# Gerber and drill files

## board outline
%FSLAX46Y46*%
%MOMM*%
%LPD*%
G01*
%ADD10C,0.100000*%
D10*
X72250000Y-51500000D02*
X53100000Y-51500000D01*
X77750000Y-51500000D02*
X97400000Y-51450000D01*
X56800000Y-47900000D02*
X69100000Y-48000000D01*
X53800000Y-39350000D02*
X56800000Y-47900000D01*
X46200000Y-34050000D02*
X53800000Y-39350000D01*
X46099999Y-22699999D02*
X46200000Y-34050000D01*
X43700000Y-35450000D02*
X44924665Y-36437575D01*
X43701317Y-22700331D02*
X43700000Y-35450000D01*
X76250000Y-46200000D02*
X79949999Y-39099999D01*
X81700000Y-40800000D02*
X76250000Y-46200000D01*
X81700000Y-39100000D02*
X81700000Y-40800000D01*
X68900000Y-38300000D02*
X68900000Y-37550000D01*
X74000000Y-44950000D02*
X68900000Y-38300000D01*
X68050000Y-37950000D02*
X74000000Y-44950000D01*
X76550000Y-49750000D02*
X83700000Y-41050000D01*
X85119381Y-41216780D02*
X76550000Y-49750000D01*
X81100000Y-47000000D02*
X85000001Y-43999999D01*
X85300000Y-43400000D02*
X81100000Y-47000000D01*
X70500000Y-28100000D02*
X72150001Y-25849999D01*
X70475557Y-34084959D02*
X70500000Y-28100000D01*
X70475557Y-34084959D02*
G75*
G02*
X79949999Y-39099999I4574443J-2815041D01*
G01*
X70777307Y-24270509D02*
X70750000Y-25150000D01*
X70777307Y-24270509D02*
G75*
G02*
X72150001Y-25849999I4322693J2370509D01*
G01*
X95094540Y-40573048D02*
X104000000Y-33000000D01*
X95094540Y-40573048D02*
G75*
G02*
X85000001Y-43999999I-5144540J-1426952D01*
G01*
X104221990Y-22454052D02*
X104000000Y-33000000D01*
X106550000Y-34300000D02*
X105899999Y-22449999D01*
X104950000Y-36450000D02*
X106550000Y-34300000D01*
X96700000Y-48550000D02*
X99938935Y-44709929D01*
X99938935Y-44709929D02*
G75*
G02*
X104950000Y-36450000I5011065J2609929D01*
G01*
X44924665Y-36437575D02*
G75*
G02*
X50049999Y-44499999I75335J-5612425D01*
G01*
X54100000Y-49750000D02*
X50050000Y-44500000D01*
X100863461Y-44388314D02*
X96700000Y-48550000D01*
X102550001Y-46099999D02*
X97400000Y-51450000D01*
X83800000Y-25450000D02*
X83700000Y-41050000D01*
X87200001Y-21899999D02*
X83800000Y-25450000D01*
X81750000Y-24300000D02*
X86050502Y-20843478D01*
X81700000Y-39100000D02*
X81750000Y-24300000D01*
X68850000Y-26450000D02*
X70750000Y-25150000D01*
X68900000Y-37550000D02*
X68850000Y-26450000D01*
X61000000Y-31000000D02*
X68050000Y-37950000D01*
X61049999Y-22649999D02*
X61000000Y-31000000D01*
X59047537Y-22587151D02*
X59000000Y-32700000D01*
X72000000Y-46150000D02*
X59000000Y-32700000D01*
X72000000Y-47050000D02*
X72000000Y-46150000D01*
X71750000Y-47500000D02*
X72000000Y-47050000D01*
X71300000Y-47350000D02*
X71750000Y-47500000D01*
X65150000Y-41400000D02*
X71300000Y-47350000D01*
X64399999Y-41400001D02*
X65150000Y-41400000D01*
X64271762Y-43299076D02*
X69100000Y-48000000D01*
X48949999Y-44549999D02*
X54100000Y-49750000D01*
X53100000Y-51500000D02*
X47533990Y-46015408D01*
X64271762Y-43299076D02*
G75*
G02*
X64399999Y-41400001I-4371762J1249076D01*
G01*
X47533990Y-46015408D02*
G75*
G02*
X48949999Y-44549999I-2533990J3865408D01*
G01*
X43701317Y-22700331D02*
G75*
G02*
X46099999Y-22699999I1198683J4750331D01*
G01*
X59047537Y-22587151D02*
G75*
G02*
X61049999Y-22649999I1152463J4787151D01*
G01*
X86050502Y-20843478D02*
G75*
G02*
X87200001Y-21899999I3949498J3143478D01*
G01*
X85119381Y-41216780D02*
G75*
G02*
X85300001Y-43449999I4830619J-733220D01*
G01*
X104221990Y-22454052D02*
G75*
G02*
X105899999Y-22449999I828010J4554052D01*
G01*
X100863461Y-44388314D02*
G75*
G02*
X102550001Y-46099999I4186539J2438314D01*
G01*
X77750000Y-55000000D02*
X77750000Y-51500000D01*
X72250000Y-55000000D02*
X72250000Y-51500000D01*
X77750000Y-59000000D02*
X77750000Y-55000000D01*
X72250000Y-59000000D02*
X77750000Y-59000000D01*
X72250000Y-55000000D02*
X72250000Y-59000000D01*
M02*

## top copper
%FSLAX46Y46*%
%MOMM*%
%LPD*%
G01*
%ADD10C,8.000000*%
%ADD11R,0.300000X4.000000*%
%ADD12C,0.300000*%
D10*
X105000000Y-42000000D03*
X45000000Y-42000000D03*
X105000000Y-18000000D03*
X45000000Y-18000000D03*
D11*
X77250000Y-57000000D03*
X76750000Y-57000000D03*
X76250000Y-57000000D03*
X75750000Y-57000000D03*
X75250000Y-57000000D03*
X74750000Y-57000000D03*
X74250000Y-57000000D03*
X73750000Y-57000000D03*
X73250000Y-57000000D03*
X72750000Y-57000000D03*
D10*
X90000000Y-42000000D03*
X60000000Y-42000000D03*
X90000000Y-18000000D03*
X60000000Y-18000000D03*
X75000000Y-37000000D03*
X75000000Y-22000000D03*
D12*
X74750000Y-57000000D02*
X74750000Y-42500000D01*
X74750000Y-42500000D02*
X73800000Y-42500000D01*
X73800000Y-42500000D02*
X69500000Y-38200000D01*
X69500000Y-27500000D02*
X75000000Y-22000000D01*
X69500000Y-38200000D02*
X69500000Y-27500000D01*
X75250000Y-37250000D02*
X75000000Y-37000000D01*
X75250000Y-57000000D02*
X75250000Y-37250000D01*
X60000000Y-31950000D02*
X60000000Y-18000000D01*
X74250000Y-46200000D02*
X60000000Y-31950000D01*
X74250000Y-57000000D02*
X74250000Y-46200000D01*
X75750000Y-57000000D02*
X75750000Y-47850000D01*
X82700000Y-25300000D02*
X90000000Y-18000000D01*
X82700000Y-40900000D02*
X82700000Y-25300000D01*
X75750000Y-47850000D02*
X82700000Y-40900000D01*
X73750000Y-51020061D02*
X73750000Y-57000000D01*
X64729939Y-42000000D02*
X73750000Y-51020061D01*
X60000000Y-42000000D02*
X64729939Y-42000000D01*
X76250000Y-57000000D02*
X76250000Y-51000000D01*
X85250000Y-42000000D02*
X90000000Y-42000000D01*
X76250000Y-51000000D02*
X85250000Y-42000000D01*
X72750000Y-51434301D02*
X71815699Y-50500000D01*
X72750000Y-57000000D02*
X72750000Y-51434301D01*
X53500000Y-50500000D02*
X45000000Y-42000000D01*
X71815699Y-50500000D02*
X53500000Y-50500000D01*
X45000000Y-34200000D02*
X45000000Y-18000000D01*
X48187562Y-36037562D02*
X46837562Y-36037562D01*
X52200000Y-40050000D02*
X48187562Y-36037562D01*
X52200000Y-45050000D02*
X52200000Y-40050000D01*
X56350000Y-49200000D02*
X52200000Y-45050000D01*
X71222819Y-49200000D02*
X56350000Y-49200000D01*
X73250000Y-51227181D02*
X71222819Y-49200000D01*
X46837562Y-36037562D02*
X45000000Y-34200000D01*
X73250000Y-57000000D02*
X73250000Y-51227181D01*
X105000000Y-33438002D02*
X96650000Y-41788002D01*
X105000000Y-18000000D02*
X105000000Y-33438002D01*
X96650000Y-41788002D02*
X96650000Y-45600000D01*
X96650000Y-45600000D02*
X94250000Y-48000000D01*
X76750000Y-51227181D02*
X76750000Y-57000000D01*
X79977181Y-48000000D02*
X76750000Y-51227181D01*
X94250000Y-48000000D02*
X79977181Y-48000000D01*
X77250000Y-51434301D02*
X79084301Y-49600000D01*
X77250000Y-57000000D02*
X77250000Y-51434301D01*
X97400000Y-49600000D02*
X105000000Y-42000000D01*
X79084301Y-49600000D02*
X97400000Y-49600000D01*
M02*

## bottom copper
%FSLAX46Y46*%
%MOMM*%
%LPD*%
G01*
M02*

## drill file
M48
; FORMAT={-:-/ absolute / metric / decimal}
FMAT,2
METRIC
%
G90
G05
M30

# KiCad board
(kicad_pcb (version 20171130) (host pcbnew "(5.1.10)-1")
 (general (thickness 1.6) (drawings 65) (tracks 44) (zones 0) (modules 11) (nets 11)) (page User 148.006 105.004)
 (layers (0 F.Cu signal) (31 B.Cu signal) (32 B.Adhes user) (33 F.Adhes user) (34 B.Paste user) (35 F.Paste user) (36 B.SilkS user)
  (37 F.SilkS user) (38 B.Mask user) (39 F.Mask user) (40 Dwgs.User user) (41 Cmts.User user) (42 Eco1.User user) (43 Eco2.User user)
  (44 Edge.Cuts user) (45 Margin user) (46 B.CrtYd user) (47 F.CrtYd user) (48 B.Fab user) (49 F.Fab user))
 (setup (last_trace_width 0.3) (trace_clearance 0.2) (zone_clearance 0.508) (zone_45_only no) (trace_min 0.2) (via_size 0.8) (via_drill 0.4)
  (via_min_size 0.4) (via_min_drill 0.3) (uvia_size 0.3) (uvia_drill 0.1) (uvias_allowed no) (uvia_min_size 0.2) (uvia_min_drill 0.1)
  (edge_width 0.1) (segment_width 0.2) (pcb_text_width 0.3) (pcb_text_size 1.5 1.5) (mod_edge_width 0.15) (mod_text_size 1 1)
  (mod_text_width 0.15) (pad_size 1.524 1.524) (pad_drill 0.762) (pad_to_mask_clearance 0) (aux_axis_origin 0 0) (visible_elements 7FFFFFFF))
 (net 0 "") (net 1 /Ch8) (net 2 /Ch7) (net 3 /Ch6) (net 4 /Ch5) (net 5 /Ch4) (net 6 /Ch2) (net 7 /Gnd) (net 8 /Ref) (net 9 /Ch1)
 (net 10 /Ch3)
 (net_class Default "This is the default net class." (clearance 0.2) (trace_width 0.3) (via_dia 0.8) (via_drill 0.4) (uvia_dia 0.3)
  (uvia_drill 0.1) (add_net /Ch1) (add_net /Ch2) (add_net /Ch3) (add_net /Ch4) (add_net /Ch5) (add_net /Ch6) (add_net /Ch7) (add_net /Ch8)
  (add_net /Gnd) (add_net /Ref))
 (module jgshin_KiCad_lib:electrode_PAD (layer F.Cu) (at 105 42)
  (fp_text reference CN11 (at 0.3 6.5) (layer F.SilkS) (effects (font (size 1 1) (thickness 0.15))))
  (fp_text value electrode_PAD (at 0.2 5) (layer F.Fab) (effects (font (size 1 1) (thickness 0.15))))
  (pad 1 smd circle (at 0 0) (size 8 8) (layers F.Cu F.Paste F.Mask) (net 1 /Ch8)))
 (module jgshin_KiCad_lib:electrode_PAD (layer F.Cu) (at 45 42)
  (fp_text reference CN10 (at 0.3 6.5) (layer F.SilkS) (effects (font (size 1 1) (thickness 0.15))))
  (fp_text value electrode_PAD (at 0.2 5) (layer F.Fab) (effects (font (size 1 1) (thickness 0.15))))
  (pad 1 smd circle (at 0 0) (size 8 8) (layers F.Cu F.Paste F.Mask) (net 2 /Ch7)))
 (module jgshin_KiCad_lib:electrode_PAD (layer F.Cu) (at 105 18)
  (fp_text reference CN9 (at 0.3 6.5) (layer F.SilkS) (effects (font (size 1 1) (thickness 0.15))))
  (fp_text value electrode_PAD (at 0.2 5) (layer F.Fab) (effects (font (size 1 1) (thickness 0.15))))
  (pad 1 smd circle (at 0 0) (size 8 8) (layers F.Cu F.Paste F.Mask) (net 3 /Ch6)))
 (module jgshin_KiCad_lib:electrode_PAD (layer F.Cu) (at 45 18)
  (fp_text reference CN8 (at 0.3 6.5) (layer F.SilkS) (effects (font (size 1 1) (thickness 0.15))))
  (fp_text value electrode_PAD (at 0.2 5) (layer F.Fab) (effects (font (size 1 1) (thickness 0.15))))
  (pad 1 smd circle (at 0 0) (size 8 8) (layers F.Cu F.Paste F.Mask) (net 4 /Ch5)))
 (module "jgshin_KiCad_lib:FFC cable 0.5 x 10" (layer F.Cu) (at 75 57)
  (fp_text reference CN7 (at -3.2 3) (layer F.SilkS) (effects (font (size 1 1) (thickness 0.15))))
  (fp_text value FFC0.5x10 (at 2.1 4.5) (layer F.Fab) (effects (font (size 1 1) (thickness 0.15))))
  (pad 10 smd rect (at 2.25 0) (size 0.3 4) (layers F.Cu F.Paste F.Mask) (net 1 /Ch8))
  (pad 9 smd rect (at 1.75 0) (size 0.3 4) (layers F.Cu F.Paste F.Mask) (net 3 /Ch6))
  (pad 8 smd rect (at 1.25 0) (size 0.3 4) (layers F.Cu F.Paste F.Mask) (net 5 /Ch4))
  (pad 7 smd rect (at 0.75 0) (size 0.3 4) (layers F.Cu F.Paste F.Mask) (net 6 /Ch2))
  (pad 6 smd rect (at 0.25 0) (size 0.3 4) (layers F.Cu F.Paste F.Mask) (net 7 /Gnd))
  (pad 5 smd rect (at -0.25 0) (size 0.3 4) (layers F.Cu F.Paste F.Mask) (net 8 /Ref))
  (pad 4 smd rect (at -0.75 0) (size 0.3 4) (layers F.Cu F.Paste F.Mask) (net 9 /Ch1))
  (pad 3 smd rect (at -1.25 0) (size 0.3 4) (layers F.Cu F.Paste F.Mask) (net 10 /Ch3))
  (pad 2 smd rect (at -1.75 0) (size 0.3 4) (layers F.Cu F.Paste F.Mask) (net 4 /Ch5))
  (pad 1 smd rect (at -2.25 0) (size 0.3 4) (layers F.Cu F.Paste F.Mask) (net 2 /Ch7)))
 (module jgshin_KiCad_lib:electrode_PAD (layer F.Cu) (at 90 42)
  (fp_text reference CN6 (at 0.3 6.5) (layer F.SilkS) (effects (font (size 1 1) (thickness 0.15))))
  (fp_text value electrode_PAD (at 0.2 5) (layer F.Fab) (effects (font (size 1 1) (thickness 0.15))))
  (pad 1 smd circle (at 0 0) (size 8 8) (layers F.Cu F.Paste F.Mask) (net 5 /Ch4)))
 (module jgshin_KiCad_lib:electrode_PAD (layer F.Cu) (at 60 42)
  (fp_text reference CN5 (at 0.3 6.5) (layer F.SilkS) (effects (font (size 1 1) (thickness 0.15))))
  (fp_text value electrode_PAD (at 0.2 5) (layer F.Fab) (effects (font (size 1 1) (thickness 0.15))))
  (pad 1 smd circle (at 0 0) (size 8 8) (layers F.Cu F.Paste F.Mask) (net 10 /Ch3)))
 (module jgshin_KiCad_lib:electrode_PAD (layer F.Cu) (at 90 18)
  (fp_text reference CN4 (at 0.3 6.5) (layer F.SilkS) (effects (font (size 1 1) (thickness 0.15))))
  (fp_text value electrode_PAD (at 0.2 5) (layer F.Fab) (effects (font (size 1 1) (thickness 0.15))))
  (pad 1 smd circle (at 0 0) (size 8 8) (layers F.Cu F.Paste F.Mask) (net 6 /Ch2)))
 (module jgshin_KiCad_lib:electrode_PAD (layer F.Cu) (at 60 18)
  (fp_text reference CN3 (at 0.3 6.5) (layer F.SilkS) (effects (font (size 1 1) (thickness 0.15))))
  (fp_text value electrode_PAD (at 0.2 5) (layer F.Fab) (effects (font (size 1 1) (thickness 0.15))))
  (pad 1 smd circle (at 0 0) (size 8 8) (layers F.Cu F.Paste F.Mask) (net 9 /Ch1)))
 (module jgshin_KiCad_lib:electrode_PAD (layer F.Cu) (at 75 37)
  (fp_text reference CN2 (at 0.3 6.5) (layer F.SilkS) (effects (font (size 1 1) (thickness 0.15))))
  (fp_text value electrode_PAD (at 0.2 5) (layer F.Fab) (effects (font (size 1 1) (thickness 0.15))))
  (pad 1 smd circle (at 0 0) (size 8 8) (layers F.Cu F.Paste F.Mask) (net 7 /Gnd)))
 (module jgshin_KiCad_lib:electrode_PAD (layer F.Cu) (at 75 22)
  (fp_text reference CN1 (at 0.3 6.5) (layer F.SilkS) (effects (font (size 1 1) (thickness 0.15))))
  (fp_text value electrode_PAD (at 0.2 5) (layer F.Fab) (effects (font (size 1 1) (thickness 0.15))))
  (pad 1 smd circle (at 0 0) (size 8 8) (layers F.Cu F.Paste F.Mask) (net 8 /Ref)))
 (gr_line (start 72.25 51.5) (end 53.1 51.5) (layer Edge.Cuts) (width 0.1))
 (gr_line (start 77.75 51.5) (end 97.4 51.45) (layer Edge.Cuts) (width 0.1))
 (gr_line (start 56.8 47.9) (end 69.1 48) (layer Edge.Cuts) (width 0.1))
 (gr_line (start 53.8 39.35) (end 56.8 47.9) (layer Edge.Cuts) (width 0.1))
 (gr_line (start 46.2 34.05) (end 53.8 39.35) (layer Edge.Cuts) (width 0.1))
 (gr_line (start 46.099999 22.699999) (end 46.2 34.05) (layer Edge.Cuts) (width 0.1))
 (gr_line (start 43.7 35.45) (end 44.924665 36.437575) (layer Edge.Cuts) (width 0.1))
 (gr_line (start 43.701317 22.700331) (end 43.7 35.45) (layer Edge.Cuts) (width 0.1))
 (gr_line (start 76.25 46.2) (end 79.949999 39.099999) (layer Edge.Cuts) (width 0.1))
 (gr_line (start 81.7 40.8) (end 76.25 46.2) (layer Edge.Cuts) (width 0.1))
 (gr_line (start 81.7 39.1) (end 81.7 40.8) (layer Edge.Cuts) (width 0.1))
 (gr_line (start 68.9 38.3) (end 68.9 37.55) (layer Edge.Cuts) (width 0.1))
 (gr_line (start 74 44.95) (end 68.9 38.3) (layer Edge.Cuts) (width 0.1))
 (gr_line (start 68.05 37.95) (end 74 44.95) (layer Edge.Cuts) (width 0.1))
 (gr_line (start 76.55 49.75) (end 83.7 41.05) (layer Edge.Cuts) (width 0.1))
 (gr_line (start 85.119381 41.21678) (end 76.55 49.75) (layer Edge.Cuts) (width 0.1))
 (gr_line (start 81.1 47) (end 85.000001 43.999999) (layer Edge.Cuts) (width 0.1))
 (gr_line (start 85.3 43.4) (end 81.1 47) (layer Edge.Cuts) (width 0.1))
 (gr_line (start 70.5 28.1) (end 72.150001 25.849999) (layer Edge.Cuts) (width 0.1))
 (gr_line (start 70.475557 34.084959) (end 70.5 28.1) (layer Edge.Cuts) (width 0.1))
 (gr_arc (start 75.05 36.9) (end 79.949999 39.099999) (angle -172.5716049) (layer Edge.Cuts) (width 0.1))
 (gr_line (start 70.777307 24.270509) (end 70.75 25.15) (layer Edge.Cuts) (width 0.1))
 (gr_arc (start 75.1 21.9) (end 72.150001 25.849999) (angle -335.4934745) (layer Edge.Cuts) (width 0.1))
 (gr_line (start 95.09454 40.573048) (end 104 33) (layer Edge.Cuts) (width 0.1))
 (gr_arc (start 89.95 42) (end 85.000001 43.999999) (angle -173.5018404) (layer Edge.Cuts) (width 0.1))
 (gr_line (start 104.22199 22.454052) (end 104 33) (layer Edge.Cuts) (width 0.1))
 (gr_line (start 106.55 34.3) (end 105.899999 22.449999) (layer Edge.Cuts) (width 0.1))
 (gr_line (start 104.95 36.45) (end 106.55 34.3) (layer Edge.Cuts) (width 0.1))
 (gr_line (start 96.7 48.55) (end 99.938935 44.709929) (layer Edge.Cuts) (width 0.1))
 (gr_arc (start 104.95 42.1) (end 104.95 36.45) (angle -117.5120026) (layer Edge.Cuts) (width 0.1))
 (gr_arc (start 45 42.05) (end 50.049999 44.499999) (angle -116.6492984) (layer Edge.Cuts) (width 0.1))
 (gr_line (start 54.1 49.75) (end 50.05 44.5) (layer Edge.Cuts) (width 0.1))
 (gr_line (start 100.863461 44.388314) (end 96.7 48.55) (layer Edge.Cuts) (width 0.1))
 (gr_line (start 102.550001 46.099999) (end 97.4 51.45) (layer Edge.Cuts) (width 0.1))
 (gr_line (start 83.8 25.45) (end 83.7 41.05) (layer Edge.Cuts) (width 0.1))
 (gr_line (start 87.200001 21.899999) (end 83.8 25.45) (layer Edge.Cuts) (width 0.1))
 (gr_line (start 81.75 24.3) (end 86.050502 20.843478) (layer Edge.Cuts) (width 0.1))
 (gr_line (start 81.7 39.1) (end 81.75 24.3) (layer Edge.Cuts) (width 0.1))
 (gr_line (start 68.85 26.45) (end 70.75 25.15) (layer Edge.Cuts) (width 0.1))
 (gr_line (start 68.9 37.55) (end 68.85 26.45) (layer Edge.Cuts) (width 0.1))
 (gr_line (start 61 31) (end 68.05 37.95) (layer Edge.Cuts) (width 0.1))
 (gr_line (start 61.049999 22.649999) (end 61 31) (layer Edge.Cuts) (width 0.1))
 (gr_line (start 59.047537 22.587151) (end 59 32.7) (layer Edge.Cuts) (width 0.1))
 (gr_line (start 72 46.15) (end 59 32.7) (layer Edge.Cuts) (width 0.1))
 (gr_line (start 72 47.05) (end 72 46.15) (layer Edge.Cuts) (width 0.1))
 (gr_line (start 71.75 47.5) (end 72 47.05) (layer Edge.Cuts) (width 0.1))
 (gr_line (start 71.3 47.35) (end 71.75 47.5) (layer Edge.Cuts) (width 0.1))
 (gr_line (start 65.15 41.4) (end 71.3 47.35) (layer Edge.Cuts) (width 0.1))
 (gr_line (start 64.399999 41.400001) (end 65.15 41.4) (layer Edge.Cuts) (width 0.1))
 (gr_line (start 64.271762 43.299076) (end 69.1 48) (layer Edge.Cuts) (width 0.1))
 (gr_line (start 48.949999 44.549999) (end 54.1 49.75) (layer Edge.Cuts) (width 0.1))
 (gr_line (start 53.1 51.5) (end 47.53399 46.015408) (layer Edge.Cuts) (width 0.1))
 (gr_arc (start 59.9 42.05) (end 64.399999 41.400001) (angle -335.8353949) (layer Edge.Cuts) (width 0.1))
 (gr_arc (start 45 42.15) (end 48.949999 44.549999) (angle -334.5297214) (layer Edge.Cuts) (width 0.1))
 (gr_arc (start 44.9 17.95) (end 46.099999 22.699999) (angle -331.6597675) (layer Edge.Cuts) (width 0.1))
 (gr_arc (start 60.2 17.8) (end 61.049999 22.649999) (angle -336.5235706) (layer Edge.Cuts) (width 0.1))
 (gr_arc (start 90 17.7) (end 87.200001 21.899999) (angle -342.2069938) (layer Edge.Cuts) (width 0.1))
 (gr_arc (start 89.95 41.95) (end 85.300001 43.449999) (angle -333.4905016) (layer Edge.Cuts) (width 0.1))
 (gr_arc (start 105.05 17.9) (end 105.899999 22.449999) (angle -339.113518) (layer Edge.Cuts) (width 0.1))
 (gr_arc (start 105.05 41.95) (end 102.550001 46.099999) (angle -331.2824388) (layer Edge.Cuts) (width 0.1))
 (gr_line (start 77.75 55) (end 77.75 51.5) (layer Edge.Cuts) (width 0.1))
 (gr_line (start 72.25 55) (end 72.25 51.5) (layer Edge.Cuts) (width 0.1))
 (gr_line (start 77.75 59) (end 77.75 55) (layer Edge.Cuts) (width 0.1))
 (gr_line (start 72.25 59) (end 77.75 59) (layer Edge.Cuts) (width 0.1))
 (gr_line (start 72.25 55) (end 72.25 59) (layer Edge.Cuts) (width 0.1))
 (segment (start 74.75 57) (end 74.75 42.5) (width 0.3) (layer F.Cu) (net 8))
 (segment (start 74.75 42.5) (end 73.8 42.5) (width 0.3) (layer F.Cu) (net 8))
 (segment (start 73.8 42.5) (end 69.5 38.2) (width 0.3) (layer F.Cu) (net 8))
 (segment (start 69.5 27.5) (end 75 22) (width 0.3) (layer F.Cu) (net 8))
 (segment (start 69.5 38.2) (end 69.5 27.5) (width 0.3) (layer F.Cu) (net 8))
 (segment (start 75.25 37.25) (end 75 37) (width 0.3) (layer F.Cu) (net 7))
 (segment (start 75.25 57) (end 75.25 37.25) (width 0.3) (layer F.Cu) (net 7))
 (segment (start 60 31.95) (end 60 18) (width 0.3) (layer F.Cu) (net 9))
 (segment (start 74.25 46.2) (end 60 31.95) (width 0.3) (layer F.Cu) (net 9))
 (segment (start 74.25 57) (end 74.25 46.2) (width 0.3) (layer F.Cu) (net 9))
 (segment (start 75.75 57) (end 75.75 47.85) (width 0.3) (layer F.Cu) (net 6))
 (segment (start 82.7 25.3) (end 90 18) (width 0.3) (layer F.Cu) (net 6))
 (segment (start 82.7 40.9) (end 82.7 25.3) (width 0.3) (layer F.Cu) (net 6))
 (segment (start 75.75 47.85) (end 82.7 40.9) (width 0.3) (layer F.Cu) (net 6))
 (segment (start 73.75 51.020061) (end 73.75 57) (width 0.3) (layer F.Cu) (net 10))
 (segment (start 64.729939 42) (end 73.75 51.020061) (width 0.3) (layer F.Cu) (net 10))
 (segment (start 60 42) (end 64.729939 42) (width 0.3) (layer F.Cu) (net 10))
 (segment (start 76.25 57) (end 76.25 51) (width 0.3) (layer F.Cu) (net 5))
 (segment (start 85.25 42) (end 90 42) (width 0.3) (layer F.Cu) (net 5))
 (segment (start 76.25 51) (end 85.25 42) (width 0.3) (layer F.Cu) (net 5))
 (segment (start 72.75 51.434301) (end 71.815699 50.5) (width 0.3) (layer F.Cu) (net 2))
 (segment (start 72.75 57) (end 72.75 51.434301) (width 0.3) (layer F.Cu) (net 2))
 (segment (start 53.5 50.5) (end 45 42) (width 0.3) (layer F.Cu) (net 2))
 (segment (start 71.815699 50.5) (end 53.5 50.5) (width 0.3) (layer F.Cu) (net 2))
 (segment (start 45 34.2) (end 45 18) (width 0.3) (layer F.Cu) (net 4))
 (segment (start 48.187562 36.037562) (end 46.837562 36.037562) (width 0.3) (layer F.Cu) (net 4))
 (segment (start 52.2 40.05) (end 48.187562 36.037562) (width 0.3) (layer F.Cu) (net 4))
 (segment (start 52.2 45.05) (end 52.2 40.05) (width 0.3) (layer F.Cu) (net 4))
 (segment (start 56.35 49.2) (end 52.2 45.05) (width 0.3) (layer F.Cu) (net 4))
 (segment (start 71.222819 49.2) (end 56.35 49.2) (width 0.3) (layer F.Cu) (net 4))
 (segment (start 73.25 51.227181) (end 71.222819 49.2) (width 0.3) (layer F.Cu) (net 4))
 (segment (start 46.837562 36.037562) (end 45 34.2) (width 0.3) (layer F.Cu) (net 4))
 (segment (start 73.25 57) (end 73.25 51.227181) (width 0.3) (layer F.Cu) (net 4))
 (segment (start 105 33.438002) (end 96.65 41.788002) (width 0.3) (layer F.Cu) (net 3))
 (segment (start 105 18) (end 105 33.438002) (width 0.3) (layer F.Cu) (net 3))
 (segment (start 96.65 41.788002) (end 96.65 45.6) (width 0.3) (layer F.Cu) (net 3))
 (segment (start 96.65 45.6) (end 94.25 48) (width 0.3) (layer F.Cu) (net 3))
 (segment (start 76.75 51.227181) (end 76.75 57) (width 0.3) (layer F.Cu) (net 3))
 (segment (start 79.977181 48) (end 76.75 51.227181) (width 0.3) (layer F.Cu) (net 3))
 (segment (start 94.25 48) (end 79.977181 48) (width 0.3) (layer F.Cu) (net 3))
 (segment (start 77.25 51.434301) (end 79.084301 49.6) (width 0.3) (layer F.Cu) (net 1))
 (segment (start 77.25 57) (end 77.25 51.434301) (width 0.3) (layer F.Cu) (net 1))
 (segment (start 97.4 49.6) (end 105 42) (width 0.3) (layer F.Cu) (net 1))
 (segment (start 79.084301 49.6) (end 97.4 49.6) (width 0.3) (layer F.Cu) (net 1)))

